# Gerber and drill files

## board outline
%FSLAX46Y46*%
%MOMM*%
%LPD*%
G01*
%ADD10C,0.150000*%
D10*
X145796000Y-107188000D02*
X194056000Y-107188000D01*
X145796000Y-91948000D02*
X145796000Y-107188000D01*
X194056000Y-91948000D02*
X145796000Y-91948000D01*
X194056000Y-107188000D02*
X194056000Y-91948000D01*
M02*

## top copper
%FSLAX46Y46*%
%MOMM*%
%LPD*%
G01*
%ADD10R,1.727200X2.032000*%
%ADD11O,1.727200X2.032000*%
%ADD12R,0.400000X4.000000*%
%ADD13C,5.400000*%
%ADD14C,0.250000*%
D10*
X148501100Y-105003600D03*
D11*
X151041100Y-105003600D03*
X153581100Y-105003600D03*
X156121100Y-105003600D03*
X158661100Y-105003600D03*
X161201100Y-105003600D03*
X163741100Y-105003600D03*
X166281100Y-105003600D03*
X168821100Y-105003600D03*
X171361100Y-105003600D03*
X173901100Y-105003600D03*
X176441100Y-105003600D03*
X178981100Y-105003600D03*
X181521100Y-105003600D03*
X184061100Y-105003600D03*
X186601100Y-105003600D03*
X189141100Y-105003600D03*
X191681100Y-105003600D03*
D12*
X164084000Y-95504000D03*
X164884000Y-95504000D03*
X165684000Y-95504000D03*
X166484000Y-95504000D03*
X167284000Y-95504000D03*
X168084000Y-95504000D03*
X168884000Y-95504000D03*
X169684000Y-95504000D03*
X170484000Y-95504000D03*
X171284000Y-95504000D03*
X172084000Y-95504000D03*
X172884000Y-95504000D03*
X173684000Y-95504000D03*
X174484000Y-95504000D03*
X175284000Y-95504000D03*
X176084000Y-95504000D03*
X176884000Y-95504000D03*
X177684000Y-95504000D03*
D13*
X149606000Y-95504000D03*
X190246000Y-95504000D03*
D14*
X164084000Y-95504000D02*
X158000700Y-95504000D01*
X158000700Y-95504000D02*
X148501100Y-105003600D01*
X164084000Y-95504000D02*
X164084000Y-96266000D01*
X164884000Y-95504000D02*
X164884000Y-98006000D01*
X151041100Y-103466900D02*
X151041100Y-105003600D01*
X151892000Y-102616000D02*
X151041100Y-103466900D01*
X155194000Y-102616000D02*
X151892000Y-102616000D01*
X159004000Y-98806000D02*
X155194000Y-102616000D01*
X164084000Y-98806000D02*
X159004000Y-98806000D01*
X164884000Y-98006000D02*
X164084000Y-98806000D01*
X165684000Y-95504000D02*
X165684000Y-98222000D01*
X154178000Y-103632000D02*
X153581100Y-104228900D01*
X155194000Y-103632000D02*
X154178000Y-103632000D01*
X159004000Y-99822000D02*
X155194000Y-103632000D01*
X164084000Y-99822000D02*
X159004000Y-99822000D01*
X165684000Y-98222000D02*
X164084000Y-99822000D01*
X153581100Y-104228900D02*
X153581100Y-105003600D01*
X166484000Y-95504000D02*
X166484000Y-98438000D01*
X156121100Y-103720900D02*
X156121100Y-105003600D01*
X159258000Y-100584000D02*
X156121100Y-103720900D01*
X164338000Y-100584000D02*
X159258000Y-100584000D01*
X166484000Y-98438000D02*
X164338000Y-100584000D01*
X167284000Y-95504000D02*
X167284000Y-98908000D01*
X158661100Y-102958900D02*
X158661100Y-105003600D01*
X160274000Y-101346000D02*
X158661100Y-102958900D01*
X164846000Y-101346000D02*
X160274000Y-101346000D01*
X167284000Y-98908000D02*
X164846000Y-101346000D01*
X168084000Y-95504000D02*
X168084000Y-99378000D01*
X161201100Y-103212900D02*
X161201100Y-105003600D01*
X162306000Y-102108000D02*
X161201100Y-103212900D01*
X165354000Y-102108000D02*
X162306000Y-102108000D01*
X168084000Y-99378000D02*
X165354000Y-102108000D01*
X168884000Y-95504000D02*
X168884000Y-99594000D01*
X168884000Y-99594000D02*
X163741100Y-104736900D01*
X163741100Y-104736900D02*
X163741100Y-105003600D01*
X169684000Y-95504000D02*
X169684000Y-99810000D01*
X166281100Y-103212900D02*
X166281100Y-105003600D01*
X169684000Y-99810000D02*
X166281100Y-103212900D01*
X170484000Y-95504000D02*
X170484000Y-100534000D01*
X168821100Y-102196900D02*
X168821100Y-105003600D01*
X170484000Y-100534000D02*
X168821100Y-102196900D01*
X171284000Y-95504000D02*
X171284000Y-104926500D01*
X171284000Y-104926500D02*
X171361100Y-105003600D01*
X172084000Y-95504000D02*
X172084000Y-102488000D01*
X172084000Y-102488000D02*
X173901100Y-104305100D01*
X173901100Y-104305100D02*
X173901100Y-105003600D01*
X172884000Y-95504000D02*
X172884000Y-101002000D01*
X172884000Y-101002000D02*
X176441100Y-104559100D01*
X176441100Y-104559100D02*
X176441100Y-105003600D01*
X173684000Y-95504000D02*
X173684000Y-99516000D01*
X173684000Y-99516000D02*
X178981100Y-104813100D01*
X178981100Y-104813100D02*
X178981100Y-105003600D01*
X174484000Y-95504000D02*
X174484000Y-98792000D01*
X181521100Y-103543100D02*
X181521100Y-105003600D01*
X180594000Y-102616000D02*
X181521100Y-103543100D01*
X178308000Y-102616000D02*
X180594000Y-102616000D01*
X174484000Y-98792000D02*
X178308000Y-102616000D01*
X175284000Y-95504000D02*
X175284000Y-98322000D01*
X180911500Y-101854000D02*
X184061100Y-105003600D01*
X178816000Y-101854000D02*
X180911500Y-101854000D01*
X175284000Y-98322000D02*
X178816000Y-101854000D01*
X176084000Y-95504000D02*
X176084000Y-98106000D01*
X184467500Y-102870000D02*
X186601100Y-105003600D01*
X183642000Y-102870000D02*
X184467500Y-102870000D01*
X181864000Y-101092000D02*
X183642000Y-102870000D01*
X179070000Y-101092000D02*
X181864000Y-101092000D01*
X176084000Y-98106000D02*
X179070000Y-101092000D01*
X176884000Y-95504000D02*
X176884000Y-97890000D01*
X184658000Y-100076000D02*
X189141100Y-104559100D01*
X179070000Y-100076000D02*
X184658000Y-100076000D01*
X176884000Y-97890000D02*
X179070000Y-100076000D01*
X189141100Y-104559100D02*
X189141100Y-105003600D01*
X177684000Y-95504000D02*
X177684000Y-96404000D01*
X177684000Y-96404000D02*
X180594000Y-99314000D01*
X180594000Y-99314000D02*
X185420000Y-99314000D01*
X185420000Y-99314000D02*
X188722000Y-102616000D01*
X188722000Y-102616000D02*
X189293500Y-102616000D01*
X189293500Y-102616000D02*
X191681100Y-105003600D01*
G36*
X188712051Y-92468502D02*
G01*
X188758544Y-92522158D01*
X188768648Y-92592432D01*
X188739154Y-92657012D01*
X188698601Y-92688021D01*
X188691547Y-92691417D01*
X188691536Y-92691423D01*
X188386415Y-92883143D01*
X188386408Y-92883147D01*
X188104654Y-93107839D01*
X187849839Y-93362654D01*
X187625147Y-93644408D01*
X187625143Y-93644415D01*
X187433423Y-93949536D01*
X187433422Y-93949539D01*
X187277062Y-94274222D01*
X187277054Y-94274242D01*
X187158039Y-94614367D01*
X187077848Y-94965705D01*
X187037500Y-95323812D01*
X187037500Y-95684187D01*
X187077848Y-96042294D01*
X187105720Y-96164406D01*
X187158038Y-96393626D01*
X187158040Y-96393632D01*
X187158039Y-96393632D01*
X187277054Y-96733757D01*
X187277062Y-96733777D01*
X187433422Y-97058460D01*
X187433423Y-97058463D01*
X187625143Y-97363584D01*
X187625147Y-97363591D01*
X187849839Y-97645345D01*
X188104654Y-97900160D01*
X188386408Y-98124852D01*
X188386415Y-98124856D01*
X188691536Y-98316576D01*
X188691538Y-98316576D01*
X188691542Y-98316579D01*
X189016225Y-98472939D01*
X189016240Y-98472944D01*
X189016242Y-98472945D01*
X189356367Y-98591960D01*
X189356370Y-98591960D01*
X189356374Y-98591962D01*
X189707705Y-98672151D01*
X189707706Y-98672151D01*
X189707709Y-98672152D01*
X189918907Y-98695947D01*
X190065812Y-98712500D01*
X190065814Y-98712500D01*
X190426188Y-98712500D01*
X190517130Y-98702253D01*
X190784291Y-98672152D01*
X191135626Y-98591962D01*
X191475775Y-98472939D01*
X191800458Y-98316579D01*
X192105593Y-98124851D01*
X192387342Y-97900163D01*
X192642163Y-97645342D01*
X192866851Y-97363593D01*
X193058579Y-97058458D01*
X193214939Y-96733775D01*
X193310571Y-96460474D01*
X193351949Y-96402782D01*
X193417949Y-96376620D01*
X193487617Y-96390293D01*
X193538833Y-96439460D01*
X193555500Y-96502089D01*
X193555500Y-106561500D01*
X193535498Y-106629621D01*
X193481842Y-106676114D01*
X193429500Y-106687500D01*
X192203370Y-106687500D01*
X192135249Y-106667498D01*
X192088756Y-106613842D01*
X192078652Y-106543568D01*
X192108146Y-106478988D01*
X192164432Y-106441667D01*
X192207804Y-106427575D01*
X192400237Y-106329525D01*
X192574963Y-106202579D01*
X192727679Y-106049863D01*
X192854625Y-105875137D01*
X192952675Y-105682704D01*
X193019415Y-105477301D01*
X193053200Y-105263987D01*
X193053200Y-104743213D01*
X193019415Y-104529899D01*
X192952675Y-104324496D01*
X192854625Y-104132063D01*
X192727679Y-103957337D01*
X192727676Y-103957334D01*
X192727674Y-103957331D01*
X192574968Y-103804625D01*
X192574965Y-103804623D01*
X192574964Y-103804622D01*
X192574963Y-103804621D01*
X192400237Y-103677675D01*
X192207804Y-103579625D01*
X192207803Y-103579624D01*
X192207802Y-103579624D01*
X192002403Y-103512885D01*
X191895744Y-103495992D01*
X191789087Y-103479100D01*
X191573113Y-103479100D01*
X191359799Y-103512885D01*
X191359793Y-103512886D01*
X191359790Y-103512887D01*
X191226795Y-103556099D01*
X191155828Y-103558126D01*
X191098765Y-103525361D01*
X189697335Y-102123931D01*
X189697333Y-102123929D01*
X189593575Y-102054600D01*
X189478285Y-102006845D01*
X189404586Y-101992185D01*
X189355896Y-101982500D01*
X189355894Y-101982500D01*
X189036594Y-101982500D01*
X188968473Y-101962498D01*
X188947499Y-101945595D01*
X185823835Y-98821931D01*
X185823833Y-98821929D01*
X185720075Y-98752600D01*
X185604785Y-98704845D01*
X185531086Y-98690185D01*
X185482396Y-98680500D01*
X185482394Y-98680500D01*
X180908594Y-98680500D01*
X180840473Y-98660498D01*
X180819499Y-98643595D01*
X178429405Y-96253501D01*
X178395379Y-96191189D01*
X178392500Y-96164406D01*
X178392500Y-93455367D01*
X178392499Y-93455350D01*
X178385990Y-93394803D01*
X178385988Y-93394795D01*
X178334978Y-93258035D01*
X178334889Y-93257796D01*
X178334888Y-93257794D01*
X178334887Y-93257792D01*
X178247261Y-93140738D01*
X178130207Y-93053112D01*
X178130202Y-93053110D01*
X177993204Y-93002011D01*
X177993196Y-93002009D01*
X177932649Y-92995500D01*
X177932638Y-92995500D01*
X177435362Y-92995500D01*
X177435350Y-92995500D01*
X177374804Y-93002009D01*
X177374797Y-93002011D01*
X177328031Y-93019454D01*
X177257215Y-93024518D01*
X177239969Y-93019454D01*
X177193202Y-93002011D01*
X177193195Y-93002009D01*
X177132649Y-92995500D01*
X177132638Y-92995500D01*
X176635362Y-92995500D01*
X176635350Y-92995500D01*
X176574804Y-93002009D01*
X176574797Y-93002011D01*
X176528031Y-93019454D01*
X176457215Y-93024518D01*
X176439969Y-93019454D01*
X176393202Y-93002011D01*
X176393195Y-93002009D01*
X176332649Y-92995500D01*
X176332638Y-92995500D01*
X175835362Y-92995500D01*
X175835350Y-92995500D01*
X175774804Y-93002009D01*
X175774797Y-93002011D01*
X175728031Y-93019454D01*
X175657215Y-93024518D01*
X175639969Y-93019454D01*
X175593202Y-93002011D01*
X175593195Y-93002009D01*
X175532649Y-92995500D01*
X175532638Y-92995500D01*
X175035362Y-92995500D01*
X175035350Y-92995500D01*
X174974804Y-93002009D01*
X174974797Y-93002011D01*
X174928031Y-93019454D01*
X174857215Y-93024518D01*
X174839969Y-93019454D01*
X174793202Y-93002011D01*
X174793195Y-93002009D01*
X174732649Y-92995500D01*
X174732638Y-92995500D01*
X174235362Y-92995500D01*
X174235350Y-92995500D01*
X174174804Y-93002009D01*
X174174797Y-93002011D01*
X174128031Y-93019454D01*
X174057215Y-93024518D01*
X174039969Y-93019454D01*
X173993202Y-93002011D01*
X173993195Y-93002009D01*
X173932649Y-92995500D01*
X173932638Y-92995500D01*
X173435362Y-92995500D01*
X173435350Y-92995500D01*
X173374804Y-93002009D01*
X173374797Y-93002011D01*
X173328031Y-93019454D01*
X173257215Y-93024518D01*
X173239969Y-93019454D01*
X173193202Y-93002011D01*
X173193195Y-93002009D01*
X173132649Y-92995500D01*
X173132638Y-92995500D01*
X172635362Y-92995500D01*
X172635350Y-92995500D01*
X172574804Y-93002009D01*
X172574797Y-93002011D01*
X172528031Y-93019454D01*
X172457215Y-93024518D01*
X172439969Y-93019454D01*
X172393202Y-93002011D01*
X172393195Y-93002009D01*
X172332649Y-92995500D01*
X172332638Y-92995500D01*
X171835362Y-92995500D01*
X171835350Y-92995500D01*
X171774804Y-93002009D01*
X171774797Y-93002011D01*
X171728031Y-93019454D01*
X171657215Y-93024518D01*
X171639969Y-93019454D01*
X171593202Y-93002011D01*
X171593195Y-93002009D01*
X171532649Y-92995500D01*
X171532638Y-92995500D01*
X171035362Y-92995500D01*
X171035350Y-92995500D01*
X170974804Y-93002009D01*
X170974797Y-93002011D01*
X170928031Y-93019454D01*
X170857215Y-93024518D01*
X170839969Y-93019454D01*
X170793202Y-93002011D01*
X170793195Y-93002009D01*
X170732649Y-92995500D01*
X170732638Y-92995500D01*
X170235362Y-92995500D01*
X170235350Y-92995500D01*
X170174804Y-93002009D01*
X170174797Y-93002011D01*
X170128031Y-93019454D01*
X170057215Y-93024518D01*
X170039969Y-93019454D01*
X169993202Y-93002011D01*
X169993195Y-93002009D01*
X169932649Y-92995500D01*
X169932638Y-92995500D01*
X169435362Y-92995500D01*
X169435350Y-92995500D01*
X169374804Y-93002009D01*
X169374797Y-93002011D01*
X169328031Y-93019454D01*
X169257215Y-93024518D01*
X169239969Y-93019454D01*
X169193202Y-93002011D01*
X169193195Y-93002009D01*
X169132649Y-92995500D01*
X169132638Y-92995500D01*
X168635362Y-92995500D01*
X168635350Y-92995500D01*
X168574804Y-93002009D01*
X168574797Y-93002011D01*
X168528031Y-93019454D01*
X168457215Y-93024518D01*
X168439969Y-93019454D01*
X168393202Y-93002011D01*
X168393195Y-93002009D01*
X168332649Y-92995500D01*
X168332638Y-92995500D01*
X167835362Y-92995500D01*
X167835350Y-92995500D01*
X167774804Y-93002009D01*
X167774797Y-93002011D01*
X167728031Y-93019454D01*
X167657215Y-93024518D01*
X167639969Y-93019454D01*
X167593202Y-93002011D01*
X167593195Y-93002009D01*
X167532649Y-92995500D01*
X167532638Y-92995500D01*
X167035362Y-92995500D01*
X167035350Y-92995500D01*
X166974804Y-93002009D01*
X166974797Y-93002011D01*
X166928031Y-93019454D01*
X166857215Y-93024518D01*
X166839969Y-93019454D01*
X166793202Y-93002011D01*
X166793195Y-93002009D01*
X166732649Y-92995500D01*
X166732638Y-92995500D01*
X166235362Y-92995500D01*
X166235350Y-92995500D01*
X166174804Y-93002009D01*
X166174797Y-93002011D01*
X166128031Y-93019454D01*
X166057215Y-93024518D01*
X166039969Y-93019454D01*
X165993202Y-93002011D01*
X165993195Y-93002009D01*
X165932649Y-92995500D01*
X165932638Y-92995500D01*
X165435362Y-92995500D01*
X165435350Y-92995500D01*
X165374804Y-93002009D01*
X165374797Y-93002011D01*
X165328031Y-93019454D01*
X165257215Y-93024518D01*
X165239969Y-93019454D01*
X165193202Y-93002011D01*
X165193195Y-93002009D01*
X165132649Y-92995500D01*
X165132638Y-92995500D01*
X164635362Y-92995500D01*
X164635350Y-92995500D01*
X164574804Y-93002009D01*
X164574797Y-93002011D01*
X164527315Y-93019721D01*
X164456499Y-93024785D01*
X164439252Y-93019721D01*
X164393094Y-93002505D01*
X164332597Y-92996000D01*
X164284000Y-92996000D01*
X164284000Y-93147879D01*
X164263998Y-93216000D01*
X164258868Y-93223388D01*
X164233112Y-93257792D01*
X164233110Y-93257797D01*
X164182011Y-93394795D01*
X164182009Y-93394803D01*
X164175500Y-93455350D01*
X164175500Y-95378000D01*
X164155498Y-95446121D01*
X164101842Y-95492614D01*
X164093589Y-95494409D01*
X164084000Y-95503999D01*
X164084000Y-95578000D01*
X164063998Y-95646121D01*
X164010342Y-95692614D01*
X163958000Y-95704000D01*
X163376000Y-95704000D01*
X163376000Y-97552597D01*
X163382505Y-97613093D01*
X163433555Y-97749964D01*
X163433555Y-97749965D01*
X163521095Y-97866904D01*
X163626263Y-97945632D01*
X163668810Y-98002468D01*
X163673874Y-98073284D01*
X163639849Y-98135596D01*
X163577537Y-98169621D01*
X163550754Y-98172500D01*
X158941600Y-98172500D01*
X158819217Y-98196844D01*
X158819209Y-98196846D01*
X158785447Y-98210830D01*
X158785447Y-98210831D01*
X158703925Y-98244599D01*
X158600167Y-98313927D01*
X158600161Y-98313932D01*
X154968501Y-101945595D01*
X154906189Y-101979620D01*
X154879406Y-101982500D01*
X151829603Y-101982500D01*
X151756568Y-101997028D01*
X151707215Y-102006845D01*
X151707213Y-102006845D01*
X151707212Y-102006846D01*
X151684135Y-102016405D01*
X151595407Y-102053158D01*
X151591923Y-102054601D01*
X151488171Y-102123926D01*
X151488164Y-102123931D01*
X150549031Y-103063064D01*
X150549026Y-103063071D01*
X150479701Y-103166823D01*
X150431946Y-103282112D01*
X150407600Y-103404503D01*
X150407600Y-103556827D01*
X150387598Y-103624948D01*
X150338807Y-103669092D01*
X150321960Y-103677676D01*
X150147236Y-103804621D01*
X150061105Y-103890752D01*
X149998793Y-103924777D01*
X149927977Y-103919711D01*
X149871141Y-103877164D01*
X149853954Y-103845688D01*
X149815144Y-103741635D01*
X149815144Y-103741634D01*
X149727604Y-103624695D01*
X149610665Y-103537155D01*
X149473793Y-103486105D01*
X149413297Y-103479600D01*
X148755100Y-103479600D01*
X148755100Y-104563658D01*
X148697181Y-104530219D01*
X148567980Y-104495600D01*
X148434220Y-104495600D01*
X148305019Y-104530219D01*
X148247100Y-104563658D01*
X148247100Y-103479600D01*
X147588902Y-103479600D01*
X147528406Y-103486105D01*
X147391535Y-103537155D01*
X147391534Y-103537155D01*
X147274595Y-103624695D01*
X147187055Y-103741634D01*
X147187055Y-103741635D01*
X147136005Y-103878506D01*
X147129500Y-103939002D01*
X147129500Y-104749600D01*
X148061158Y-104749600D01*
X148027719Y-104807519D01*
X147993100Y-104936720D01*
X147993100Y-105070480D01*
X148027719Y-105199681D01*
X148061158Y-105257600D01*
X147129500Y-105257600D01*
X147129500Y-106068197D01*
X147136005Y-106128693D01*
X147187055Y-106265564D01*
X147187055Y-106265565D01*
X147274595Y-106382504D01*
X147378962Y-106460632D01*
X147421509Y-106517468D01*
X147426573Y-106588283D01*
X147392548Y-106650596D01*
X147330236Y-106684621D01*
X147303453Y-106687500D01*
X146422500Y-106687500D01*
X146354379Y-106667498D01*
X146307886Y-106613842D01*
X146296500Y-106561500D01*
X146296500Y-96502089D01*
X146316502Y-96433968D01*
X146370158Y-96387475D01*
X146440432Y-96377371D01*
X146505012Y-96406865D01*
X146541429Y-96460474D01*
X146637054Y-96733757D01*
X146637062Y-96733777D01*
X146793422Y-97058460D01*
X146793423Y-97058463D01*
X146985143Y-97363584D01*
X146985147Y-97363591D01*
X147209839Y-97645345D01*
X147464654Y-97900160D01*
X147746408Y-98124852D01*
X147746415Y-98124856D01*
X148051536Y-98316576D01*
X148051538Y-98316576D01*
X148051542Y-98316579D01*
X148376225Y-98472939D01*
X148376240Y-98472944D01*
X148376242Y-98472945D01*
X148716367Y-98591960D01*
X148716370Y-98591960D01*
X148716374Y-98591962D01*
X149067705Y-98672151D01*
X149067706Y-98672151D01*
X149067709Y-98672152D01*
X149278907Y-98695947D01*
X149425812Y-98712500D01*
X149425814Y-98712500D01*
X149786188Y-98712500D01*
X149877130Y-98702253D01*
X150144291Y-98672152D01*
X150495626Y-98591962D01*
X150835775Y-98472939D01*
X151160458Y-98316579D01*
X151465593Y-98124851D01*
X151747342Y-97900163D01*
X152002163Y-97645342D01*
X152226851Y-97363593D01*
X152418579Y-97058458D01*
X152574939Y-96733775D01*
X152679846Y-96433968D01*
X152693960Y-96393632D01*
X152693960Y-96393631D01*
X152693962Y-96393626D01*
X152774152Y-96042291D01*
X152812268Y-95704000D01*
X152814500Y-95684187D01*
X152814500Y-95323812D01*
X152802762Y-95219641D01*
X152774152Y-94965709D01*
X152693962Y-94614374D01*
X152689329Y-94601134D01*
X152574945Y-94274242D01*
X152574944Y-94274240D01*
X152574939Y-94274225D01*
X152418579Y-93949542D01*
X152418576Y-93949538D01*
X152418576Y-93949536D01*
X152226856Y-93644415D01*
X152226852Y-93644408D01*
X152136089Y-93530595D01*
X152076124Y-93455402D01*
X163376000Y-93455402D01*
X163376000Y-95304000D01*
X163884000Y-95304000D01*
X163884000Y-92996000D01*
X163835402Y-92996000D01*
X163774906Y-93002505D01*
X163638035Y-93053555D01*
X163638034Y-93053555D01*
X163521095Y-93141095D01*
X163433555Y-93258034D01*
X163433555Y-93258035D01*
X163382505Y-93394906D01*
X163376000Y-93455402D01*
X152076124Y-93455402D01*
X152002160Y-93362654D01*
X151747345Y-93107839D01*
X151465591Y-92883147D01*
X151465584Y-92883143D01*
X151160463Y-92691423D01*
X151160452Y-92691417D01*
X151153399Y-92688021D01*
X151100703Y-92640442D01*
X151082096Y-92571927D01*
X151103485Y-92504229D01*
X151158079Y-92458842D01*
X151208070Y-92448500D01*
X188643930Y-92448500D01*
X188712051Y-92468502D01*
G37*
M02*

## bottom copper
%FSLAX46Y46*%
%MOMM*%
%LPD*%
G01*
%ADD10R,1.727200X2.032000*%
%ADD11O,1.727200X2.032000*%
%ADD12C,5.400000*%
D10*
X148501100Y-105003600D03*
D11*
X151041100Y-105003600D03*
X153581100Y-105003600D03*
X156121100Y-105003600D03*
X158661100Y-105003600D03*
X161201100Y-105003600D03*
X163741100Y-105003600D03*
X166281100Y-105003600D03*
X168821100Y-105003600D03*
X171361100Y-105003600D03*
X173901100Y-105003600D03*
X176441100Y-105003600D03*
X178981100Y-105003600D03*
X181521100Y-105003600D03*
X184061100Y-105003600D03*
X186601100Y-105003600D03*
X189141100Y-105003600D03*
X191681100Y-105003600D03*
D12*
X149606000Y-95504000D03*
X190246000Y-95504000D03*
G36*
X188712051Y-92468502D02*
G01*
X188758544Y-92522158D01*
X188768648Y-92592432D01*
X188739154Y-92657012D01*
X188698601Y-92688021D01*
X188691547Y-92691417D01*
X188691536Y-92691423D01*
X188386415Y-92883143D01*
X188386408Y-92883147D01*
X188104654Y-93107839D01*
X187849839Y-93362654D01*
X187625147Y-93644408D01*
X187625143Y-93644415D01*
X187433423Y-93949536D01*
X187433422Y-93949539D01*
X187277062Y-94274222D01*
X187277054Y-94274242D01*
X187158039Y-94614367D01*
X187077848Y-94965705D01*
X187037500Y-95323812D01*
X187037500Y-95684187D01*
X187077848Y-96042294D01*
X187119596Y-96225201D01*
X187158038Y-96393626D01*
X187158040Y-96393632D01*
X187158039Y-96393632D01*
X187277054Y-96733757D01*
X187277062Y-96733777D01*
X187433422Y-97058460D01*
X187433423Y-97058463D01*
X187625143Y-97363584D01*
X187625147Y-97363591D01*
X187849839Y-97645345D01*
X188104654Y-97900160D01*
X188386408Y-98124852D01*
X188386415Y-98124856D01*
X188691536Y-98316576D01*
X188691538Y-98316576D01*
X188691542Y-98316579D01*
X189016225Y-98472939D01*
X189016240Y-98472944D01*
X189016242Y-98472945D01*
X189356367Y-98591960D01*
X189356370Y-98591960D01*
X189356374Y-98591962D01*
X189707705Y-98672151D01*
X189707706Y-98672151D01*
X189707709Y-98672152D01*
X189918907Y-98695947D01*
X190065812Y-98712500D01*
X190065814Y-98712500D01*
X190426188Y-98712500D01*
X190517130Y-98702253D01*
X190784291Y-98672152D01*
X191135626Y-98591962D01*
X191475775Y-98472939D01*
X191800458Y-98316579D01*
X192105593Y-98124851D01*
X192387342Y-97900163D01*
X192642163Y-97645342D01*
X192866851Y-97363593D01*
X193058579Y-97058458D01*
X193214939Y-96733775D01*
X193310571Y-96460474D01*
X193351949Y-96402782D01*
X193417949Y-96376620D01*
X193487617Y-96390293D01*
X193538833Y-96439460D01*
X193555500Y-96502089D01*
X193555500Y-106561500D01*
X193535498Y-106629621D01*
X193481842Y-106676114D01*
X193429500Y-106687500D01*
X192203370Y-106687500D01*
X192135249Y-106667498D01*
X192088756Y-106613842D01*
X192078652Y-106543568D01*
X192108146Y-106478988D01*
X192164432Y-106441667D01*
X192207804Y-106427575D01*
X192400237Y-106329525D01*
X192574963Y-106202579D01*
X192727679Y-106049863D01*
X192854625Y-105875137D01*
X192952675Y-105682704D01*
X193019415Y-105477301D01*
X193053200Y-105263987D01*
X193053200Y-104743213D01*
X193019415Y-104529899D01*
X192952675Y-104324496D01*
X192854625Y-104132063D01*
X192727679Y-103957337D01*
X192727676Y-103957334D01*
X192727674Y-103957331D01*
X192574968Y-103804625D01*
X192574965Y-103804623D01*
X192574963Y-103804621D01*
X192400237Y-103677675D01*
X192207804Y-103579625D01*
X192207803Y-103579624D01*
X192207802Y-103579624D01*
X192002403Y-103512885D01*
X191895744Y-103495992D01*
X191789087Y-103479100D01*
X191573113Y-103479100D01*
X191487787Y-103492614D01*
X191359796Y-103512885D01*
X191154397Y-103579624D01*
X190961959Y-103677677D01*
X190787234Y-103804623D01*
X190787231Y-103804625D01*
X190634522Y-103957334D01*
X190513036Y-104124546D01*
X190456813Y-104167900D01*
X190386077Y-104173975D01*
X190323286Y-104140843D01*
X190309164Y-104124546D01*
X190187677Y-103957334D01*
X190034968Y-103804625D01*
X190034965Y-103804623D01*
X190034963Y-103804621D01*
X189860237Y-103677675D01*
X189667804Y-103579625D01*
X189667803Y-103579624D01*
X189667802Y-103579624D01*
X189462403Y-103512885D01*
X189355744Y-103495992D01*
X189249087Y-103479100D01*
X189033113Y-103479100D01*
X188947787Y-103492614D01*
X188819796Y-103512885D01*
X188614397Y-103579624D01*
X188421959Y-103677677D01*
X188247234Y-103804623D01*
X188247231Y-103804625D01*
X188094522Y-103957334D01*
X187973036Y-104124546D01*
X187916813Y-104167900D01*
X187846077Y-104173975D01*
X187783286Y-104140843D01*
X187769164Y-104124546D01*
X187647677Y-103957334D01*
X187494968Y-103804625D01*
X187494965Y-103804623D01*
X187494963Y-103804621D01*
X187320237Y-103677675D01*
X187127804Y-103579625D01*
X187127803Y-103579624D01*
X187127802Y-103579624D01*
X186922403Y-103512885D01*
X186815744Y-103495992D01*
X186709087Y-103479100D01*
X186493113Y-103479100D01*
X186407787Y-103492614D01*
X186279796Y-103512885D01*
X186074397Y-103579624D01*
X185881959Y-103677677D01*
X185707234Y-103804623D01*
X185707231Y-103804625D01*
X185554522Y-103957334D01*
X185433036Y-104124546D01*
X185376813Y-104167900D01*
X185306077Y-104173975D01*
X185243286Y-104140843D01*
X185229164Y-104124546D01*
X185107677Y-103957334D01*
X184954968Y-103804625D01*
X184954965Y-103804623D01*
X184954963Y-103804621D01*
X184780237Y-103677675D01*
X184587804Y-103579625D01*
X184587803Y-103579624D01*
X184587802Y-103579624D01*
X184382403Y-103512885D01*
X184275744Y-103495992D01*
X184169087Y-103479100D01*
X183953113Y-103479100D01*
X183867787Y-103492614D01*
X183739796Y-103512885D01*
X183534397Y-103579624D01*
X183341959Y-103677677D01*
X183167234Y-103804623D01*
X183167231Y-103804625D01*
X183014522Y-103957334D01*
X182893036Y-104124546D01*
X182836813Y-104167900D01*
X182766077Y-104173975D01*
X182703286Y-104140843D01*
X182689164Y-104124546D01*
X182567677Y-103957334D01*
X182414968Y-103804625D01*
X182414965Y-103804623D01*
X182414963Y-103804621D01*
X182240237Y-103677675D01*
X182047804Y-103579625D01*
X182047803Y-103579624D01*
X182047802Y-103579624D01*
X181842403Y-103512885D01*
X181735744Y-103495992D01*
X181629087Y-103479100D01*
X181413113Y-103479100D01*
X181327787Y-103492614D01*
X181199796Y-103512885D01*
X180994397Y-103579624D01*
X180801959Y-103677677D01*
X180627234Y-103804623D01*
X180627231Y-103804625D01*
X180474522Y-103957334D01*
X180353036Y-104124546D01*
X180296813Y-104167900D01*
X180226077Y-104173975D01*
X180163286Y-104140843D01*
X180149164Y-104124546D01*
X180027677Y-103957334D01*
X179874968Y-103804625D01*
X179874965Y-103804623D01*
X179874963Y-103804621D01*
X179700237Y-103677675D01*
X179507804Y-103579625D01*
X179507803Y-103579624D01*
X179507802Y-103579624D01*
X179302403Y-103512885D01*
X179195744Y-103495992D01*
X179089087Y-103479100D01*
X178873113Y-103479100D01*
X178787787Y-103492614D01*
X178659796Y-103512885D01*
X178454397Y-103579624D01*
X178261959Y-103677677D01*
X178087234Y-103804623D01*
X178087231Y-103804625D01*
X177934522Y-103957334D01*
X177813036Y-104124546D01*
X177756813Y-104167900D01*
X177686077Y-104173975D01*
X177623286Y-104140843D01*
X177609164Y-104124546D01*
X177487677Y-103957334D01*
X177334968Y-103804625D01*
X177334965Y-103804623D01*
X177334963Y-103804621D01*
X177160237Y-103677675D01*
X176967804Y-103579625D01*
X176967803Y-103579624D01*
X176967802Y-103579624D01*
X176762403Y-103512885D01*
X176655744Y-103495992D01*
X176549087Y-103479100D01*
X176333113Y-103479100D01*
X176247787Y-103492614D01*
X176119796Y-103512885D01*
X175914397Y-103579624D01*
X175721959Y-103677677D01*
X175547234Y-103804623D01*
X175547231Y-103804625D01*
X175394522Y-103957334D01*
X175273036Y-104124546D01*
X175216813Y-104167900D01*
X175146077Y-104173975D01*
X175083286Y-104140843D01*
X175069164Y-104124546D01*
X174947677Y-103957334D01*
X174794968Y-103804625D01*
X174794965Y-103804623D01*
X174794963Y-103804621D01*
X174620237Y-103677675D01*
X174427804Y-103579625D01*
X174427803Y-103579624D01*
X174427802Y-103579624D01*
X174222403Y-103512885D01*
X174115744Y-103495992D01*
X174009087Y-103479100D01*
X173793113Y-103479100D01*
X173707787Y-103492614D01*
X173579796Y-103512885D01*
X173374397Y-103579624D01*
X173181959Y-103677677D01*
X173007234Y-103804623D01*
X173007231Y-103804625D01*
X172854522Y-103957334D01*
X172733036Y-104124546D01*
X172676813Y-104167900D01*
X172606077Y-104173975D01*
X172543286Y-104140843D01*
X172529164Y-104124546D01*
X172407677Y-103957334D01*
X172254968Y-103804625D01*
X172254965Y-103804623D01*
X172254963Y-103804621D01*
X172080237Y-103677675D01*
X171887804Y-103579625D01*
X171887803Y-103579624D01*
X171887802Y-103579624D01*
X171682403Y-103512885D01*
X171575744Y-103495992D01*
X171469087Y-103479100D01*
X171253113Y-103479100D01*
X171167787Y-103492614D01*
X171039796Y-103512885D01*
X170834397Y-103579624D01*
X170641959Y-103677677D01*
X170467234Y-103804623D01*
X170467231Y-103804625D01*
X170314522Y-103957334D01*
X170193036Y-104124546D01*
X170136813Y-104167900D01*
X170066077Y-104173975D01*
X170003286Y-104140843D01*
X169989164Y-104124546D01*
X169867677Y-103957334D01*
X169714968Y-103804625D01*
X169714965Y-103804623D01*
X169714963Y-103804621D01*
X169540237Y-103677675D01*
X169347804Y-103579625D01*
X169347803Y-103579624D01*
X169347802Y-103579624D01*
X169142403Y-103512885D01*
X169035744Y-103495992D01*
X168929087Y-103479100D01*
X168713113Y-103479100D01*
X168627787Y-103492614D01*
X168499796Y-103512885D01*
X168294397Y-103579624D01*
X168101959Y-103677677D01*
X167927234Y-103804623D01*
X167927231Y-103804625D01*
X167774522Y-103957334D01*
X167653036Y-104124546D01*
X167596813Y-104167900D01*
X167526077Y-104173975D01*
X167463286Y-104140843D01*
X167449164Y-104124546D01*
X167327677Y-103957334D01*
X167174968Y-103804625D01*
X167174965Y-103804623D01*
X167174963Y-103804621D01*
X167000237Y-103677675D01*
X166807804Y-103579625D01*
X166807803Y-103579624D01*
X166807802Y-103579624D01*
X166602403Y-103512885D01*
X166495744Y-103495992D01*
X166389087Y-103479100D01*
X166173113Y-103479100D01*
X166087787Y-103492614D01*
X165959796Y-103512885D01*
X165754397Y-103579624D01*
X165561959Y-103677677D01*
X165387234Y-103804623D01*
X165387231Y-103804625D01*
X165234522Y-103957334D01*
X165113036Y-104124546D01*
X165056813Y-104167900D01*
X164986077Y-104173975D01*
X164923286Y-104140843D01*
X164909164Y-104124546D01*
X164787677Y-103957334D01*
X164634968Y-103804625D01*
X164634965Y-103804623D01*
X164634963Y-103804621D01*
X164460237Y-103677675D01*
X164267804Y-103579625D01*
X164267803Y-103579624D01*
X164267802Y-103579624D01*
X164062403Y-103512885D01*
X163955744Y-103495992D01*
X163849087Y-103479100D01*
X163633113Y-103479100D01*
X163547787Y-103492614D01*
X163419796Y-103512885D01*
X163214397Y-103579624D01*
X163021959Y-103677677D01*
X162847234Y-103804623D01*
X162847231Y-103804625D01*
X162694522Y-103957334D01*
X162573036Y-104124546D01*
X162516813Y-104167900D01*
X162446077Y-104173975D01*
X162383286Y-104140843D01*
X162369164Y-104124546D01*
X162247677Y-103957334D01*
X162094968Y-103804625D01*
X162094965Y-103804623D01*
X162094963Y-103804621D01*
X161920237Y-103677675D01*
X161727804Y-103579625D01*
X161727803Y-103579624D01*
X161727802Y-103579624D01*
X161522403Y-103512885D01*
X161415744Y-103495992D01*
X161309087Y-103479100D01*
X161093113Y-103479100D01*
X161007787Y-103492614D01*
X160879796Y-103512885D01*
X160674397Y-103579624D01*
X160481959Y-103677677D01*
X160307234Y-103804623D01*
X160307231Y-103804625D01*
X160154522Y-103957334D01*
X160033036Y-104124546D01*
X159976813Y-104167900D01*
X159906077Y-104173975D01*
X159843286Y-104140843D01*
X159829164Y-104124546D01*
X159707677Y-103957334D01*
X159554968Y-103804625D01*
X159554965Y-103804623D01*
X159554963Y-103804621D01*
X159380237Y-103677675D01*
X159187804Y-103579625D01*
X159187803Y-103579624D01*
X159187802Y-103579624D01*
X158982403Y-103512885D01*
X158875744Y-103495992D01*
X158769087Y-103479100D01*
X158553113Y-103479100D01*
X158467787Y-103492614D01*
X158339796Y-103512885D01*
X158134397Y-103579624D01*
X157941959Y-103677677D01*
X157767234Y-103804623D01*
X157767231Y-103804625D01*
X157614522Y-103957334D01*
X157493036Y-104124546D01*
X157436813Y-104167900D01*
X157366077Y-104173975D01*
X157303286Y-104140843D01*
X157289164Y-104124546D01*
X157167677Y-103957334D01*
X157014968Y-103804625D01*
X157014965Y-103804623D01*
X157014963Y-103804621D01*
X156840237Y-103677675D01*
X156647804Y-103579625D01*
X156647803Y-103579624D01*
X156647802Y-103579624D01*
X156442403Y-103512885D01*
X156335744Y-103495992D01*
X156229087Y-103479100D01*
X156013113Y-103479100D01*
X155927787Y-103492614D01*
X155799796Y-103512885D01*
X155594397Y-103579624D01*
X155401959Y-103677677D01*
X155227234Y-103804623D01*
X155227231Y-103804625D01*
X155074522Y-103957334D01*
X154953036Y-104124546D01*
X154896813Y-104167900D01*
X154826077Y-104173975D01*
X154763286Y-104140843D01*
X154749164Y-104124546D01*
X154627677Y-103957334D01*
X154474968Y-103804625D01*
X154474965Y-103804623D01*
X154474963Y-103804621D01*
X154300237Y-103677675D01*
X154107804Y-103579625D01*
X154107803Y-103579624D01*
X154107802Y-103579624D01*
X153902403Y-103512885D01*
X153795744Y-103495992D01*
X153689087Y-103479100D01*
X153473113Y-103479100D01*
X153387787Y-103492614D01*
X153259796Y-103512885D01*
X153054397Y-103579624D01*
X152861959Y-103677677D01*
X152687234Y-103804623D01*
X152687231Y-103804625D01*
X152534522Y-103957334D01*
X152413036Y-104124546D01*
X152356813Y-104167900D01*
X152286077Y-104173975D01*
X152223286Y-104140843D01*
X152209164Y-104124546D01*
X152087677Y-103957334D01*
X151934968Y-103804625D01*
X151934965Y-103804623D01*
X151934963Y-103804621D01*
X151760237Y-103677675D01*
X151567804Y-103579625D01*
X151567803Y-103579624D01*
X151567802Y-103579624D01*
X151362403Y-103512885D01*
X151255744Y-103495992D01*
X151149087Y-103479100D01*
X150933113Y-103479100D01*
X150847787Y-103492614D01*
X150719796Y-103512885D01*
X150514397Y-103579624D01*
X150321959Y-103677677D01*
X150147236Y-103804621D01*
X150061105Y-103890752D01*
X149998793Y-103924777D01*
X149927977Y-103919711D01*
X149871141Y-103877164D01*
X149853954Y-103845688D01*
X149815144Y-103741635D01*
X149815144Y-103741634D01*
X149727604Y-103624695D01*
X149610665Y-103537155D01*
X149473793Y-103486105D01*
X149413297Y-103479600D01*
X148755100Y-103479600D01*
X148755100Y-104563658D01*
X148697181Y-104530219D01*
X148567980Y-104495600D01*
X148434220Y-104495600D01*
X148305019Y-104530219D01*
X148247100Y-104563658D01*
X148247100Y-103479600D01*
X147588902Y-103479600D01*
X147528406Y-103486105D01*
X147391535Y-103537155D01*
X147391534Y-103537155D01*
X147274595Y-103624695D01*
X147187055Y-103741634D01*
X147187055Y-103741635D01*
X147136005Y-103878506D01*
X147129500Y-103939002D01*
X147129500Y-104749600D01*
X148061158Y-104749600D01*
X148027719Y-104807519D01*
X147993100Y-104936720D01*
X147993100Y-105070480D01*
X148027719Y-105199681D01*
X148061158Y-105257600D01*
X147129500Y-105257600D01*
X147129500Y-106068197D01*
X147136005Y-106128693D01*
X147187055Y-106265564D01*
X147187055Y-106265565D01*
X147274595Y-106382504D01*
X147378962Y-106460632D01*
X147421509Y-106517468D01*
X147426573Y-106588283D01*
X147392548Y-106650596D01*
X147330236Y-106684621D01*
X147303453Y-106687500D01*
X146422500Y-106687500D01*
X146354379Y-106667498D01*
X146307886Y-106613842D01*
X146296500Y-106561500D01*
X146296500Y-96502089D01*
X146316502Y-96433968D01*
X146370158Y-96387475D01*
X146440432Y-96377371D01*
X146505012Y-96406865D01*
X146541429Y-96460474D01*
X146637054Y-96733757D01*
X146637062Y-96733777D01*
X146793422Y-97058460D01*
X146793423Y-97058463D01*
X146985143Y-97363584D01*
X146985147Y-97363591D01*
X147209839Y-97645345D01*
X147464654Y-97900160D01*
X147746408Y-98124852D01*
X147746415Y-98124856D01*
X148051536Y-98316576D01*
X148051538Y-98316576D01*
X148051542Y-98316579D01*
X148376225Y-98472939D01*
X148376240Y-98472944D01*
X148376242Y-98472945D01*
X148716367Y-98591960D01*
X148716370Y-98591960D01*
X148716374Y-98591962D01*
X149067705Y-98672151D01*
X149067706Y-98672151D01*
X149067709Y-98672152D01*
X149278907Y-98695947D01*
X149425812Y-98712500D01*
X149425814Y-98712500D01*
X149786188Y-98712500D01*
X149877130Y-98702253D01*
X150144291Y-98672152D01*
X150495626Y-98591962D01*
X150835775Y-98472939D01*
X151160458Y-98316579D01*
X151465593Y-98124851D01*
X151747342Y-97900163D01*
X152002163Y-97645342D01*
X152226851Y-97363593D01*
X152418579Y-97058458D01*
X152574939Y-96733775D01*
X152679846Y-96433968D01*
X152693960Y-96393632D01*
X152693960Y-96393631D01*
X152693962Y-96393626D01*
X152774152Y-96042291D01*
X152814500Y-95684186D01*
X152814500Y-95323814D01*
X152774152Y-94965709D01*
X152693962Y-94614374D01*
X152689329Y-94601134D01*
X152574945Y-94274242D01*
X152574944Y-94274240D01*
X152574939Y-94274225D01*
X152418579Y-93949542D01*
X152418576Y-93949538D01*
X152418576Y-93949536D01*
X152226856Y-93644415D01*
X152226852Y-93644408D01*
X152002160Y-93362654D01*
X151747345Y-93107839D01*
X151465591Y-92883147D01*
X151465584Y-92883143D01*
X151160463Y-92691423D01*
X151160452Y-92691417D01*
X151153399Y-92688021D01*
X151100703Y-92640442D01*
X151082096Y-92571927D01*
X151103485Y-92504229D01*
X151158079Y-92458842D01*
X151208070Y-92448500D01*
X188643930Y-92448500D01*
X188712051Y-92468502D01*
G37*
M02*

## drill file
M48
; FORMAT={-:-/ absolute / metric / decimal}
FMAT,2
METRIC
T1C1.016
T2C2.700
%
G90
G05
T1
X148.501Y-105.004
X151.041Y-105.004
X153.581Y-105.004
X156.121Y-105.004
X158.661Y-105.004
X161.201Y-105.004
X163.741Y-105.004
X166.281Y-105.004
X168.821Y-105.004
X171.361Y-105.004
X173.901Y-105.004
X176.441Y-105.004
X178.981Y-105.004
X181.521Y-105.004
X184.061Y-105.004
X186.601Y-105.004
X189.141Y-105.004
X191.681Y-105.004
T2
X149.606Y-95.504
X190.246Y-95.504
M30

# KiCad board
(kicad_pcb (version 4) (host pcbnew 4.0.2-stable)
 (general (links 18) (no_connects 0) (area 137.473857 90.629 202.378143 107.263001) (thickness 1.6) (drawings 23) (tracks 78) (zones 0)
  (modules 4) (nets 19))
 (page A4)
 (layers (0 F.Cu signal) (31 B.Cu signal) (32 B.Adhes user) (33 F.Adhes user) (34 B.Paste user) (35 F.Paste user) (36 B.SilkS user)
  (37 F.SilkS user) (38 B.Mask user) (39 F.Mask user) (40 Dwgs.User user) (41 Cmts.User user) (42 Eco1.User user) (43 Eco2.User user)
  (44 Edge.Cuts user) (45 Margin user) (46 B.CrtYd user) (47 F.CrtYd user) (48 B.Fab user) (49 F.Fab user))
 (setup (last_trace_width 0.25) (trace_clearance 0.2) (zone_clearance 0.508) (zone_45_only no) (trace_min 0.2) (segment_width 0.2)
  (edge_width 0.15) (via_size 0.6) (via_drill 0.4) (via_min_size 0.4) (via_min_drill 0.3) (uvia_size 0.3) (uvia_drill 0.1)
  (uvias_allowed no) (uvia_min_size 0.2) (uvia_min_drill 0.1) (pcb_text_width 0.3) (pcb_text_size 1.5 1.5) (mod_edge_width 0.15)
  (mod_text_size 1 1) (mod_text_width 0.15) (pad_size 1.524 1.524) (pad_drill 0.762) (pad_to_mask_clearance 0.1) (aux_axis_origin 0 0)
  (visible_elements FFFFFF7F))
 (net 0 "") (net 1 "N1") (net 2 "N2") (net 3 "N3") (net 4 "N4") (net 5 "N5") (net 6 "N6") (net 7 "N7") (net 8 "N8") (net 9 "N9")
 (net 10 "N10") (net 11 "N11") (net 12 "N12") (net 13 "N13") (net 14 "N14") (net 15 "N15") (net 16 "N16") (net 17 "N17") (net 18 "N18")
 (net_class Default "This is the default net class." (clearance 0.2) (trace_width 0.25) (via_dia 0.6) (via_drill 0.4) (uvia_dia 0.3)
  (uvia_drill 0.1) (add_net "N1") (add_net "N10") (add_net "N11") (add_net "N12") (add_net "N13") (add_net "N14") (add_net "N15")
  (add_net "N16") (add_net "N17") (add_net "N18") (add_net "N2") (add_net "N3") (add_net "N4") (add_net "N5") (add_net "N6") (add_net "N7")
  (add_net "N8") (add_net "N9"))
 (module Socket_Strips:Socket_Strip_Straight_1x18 (layer F.Cu) (at 148.5011 105.0036)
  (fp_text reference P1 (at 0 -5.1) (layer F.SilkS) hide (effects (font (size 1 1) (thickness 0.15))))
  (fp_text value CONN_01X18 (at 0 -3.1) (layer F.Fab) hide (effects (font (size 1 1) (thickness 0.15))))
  (pad 1 thru_hole rect (at 0 0) (size 1.7272 2.032) (drill 1.016) (layers *.Cu *.Mask) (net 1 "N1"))
  (pad 2 thru_hole oval (at 2.54 0) (size 1.7272 2.032) (drill 1.016) (layers *.Cu *.Mask) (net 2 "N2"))
  (pad 3 thru_hole oval (at 5.08 0) (size 1.7272 2.032) (drill 1.016) (layers *.Cu *.Mask) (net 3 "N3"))
  (pad 4 thru_hole oval (at 7.62 0) (size 1.7272 2.032) (drill 1.016) (layers *.Cu *.Mask) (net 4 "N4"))
  (pad 5 thru_hole oval (at 10.16 0) (size 1.7272 2.032) (drill 1.016) (layers *.Cu *.Mask) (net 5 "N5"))
  (pad 6 thru_hole oval (at 12.7 0) (size 1.7272 2.032) (drill 1.016) (layers *.Cu *.Mask) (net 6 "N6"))
  (pad 7 thru_hole oval (at 15.24 0) (size 1.7272 2.032) (drill 1.016) (layers *.Cu *.Mask) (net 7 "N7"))
  (pad 8 thru_hole oval (at 17.78 0) (size 1.7272 2.032) (drill 1.016) (layers *.Cu *.Mask) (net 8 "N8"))
  (pad 9 thru_hole oval (at 20.32 0) (size 1.7272 2.032) (drill 1.016) (layers *.Cu *.Mask) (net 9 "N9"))
  (pad 10 thru_hole oval (at 22.86 0) (size 1.7272 2.032) (drill 1.016) (layers *.Cu *.Mask) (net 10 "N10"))
  (pad 11 thru_hole oval (at 25.4 0) (size 1.7272 2.032) (drill 1.016) (layers *.Cu *.Mask) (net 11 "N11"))
  (pad 12 thru_hole oval (at 27.94 0) (size 1.7272 2.032) (drill 1.016) (layers *.Cu *.Mask) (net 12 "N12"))
  (pad 13 thru_hole oval (at 30.48 0) (size 1.7272 2.032) (drill 1.016) (layers *.Cu *.Mask) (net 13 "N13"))
  (pad 14 thru_hole oval (at 33.02 0) (size 1.7272 2.032) (drill 1.016) (layers *.Cu *.Mask) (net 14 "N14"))
  (pad 15 thru_hole oval (at 35.56 0) (size 1.7272 2.032) (drill 1.016) (layers *.Cu *.Mask) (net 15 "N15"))
  (pad 16 thru_hole oval (at 38.1 0) (size 1.7272 2.032) (drill 1.016) (layers *.Cu *.Mask) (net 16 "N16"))
  (pad 17 thru_hole oval (at 40.64 0) (size 1.7272 2.032) (drill 1.016) (layers *.Cu *.Mask) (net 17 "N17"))
  (pad 18 thru_hole oval (at 43.18 0) (size 1.7272 2.032) (drill 1.016) (layers *.Cu *.Mask) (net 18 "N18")))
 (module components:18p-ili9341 (layer F.Cu) (at 164.084 95.504)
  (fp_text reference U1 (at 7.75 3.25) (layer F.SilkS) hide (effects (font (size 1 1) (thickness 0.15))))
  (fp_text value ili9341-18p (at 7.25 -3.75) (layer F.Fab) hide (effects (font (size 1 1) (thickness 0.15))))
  (pad 1 smd rect (at 0 0) (size 0.4 4) (layers F.Cu F.Paste F.Mask) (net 1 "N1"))
  (pad 2 smd rect (at 0.8 0) (size 0.4 4) (layers F.Cu F.Paste F.Mask) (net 2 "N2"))
  (pad 3 smd rect (at 1.6 0) (size 0.4 4) (layers F.Cu F.Paste F.Mask) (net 3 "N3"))
  (pad 4 smd rect (at 2.4 0) (size 0.4 4) (layers F.Cu F.Paste F.Mask) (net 4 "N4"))
  (pad 5 smd rect (at 3.2 0) (size 0.4 4) (layers F.Cu F.Paste F.Mask) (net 5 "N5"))
  (pad 6 smd rect (at 4 0) (size 0.4 4) (layers F.Cu F.Paste F.Mask) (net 6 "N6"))
  (pad 7 smd rect (at 4.8 0) (size 0.4 4) (layers F.Cu F.Paste F.Mask) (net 7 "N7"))
  (pad 8 smd rect (at 5.6 0) (size 0.4 4) (layers F.Cu F.Paste F.Mask) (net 8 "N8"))
  (pad 9 smd rect (at 6.4 0) (size 0.4 4) (layers F.Cu F.Paste F.Mask) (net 9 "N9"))
  (pad 10 smd rect (at 7.2 0) (size 0.4 4) (layers F.Cu F.Paste F.Mask) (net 10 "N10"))
  (pad 11 smd rect (at 8 0) (size 0.4 4) (layers F.Cu F.Paste F.Mask) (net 11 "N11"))
  (pad 12 smd rect (at 8.8 0) (size 0.4 4) (layers F.Cu F.Paste F.Mask) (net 12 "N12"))
  (pad 13 smd rect (at 9.6 0) (size 0.4 4) (layers F.Cu F.Paste F.Mask) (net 13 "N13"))
  (pad 14 smd rect (at 10.4 0) (size 0.4 4) (layers F.Cu F.Paste F.Mask) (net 14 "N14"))
  (pad 15 smd rect (at 11.2 0) (size 0.4 4) (layers F.Cu F.Paste F.Mask) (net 15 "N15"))
  (pad 16 smd rect (at 12 0) (size 0.4 4) (layers F.Cu F.Paste F.Mask) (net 16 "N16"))
  (pad 17 smd rect (at 12.8 0) (size 0.4 4) (layers F.Cu F.Paste F.Mask) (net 17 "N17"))
  (pad 18 smd rect (at 13.6 0) (size 0.4 4) (layers F.Cu F.Paste F.Mask) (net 18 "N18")))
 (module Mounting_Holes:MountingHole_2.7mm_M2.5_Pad (layer F.Cu) (at 149.606 95.504)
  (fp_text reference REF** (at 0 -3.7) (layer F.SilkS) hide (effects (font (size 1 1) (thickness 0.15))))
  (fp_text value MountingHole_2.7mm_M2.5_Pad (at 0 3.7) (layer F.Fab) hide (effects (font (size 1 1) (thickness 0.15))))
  (pad 1 thru_hole circle (at 0 0) (size 5.4 5.4) (drill 2.7) (layers *.Cu *.Mask)))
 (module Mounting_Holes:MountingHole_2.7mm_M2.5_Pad (layer F.Cu) (at 190.246 95.504)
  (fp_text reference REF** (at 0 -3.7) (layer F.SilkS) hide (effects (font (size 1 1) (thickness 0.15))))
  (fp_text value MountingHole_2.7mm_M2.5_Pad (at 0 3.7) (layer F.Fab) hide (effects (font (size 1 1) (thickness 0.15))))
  (pad 1 thru_hole circle (at 0 0) (size 5.4 5.4) (drill 2.7) (layers *.Cu *.Mask)))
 (gr_line (start 145.796 107.188) (end 194.056 107.188) (angle 90) (layer Edge.Cuts) (width 0.15))
 (gr_line (start 145.796 91.948) (end 145.796 107.188) (angle 90) (layer Edge.Cuts) (width 0.15))
 (gr_line (start 194.056 91.948) (end 145.796 91.948) (angle 90) (layer Edge.Cuts) (width 0.15))
 (gr_line (start 194.056 107.188) (end 194.056 91.948) (angle 90) (layer Edge.Cuts) (width 0.15))
 (segment (start 164.084 95.504) (end 158.0007 95.504) (width 0.25) (layer F.Cu) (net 1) (status 400000))
 (segment (start 158.0007 95.504) (end 148.5011 105.0036) (width 0.25) (layer F.Cu) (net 1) (status 800000))
 (segment (start 164.084 95.504) (end 164.084 96.266) (width 0.25) (layer F.Cu) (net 1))
 (segment (start 164.884 95.504) (end 164.884 98.006) (width 0.25) (layer F.Cu) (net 2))
 (segment (start 151.0411 103.4669) (end 151.0411 105.0036) (width 0.25) (layer F.Cu) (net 2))
 (segment (start 151.892 102.616) (end 151.0411 103.4669) (width 0.25) (layer F.Cu) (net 2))
 (segment (start 155.194 102.616) (end 151.892 102.616) (width 0.25) (layer F.Cu) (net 2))
 (segment (start 159.004 98.806) (end 155.194 102.616) (width 0.25) (layer F.Cu) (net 2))
 (segment (start 164.084 98.806) (end 159.004 98.806) (width 0.25) (layer F.Cu) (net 2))
 (segment (start 164.884 98.006) (end 164.084 98.806) (width 0.25) (layer F.Cu) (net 2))
 (segment (start 165.684 95.504) (end 165.684 98.222) (width 0.25) (layer F.Cu) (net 3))
 (segment (start 154.178 103.632) (end 153.5811 104.2289) (width 0.25) (layer F.Cu) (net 3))
 (segment (start 155.194 103.632) (end 154.178 103.632) (width 0.25) (layer F.Cu) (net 3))
 (segment (start 159.004 99.822) (end 155.194 103.632) (width 0.25) (layer F.Cu) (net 3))
 (segment (start 164.084 99.822) (end 159.004 99.822) (width 0.25) (layer F.Cu) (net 3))
 (segment (start 165.684 98.222) (end 164.084 99.822) (width 0.25) (layer F.Cu) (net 3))
 (segment (start 153.5811 104.2289) (end 153.5811 105.0036) (width 0.25) (layer F.Cu) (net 3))
 (segment (start 166.484 95.504) (end 166.484 98.438) (width 0.25) (layer F.Cu) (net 4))
 (segment (start 156.1211 103.7209) (end 156.1211 105.0036) (width 0.25) (layer F.Cu) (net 4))
 (segment (start 159.258 100.584) (end 156.1211 103.7209) (width 0.25) (layer F.Cu) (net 4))
 (segment (start 164.338 100.584) (end 159.258 100.584) (width 0.25) (layer F.Cu) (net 4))
 (segment (start 166.484 98.438) (end 164.338 100.584) (width 0.25) (layer F.Cu) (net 4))
 (segment (start 167.284 95.504) (end 167.284 98.908) (width 0.25) (layer F.Cu) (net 5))
 (segment (start 158.6611 102.9589) (end 158.6611 105.0036) (width 0.25) (layer F.Cu) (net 5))
 (segment (start 160.274 101.346) (end 158.6611 102.9589) (width 0.25) (layer F.Cu) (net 5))
 (segment (start 164.846 101.346) (end 160.274 101.346) (width 0.25) (layer F.Cu) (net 5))
 (segment (start 167.284 98.908) (end 164.846 101.346) (width 0.25) (layer F.Cu) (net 5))
 (segment (start 168.084 95.504) (end 168.084 99.378) (width 0.25) (layer F.Cu) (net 6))
 (segment (start 161.2011 103.2129) (end 161.2011 105.0036) (width 0.25) (layer F.Cu) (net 6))
 (segment (start 162.306 102.108) (end 161.2011 103.2129) (width 0.25) (layer F.Cu) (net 6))
 (segment (start 165.354 102.108) (end 162.306 102.108) (width 0.25) (layer F.Cu) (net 6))
 (segment (start 168.084 99.378) (end 165.354 102.108) (width 0.25) (layer F.Cu) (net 6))
 (segment (start 168.884 95.504) (end 168.884 99.594) (width 0.25) (layer F.Cu) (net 7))
 (segment (start 168.884 99.594) (end 163.7411 104.7369) (width 0.25) (layer F.Cu) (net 7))
 (segment (start 163.7411 104.7369) (end 163.7411 105.0036) (width 0.25) (layer F.Cu) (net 7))
 (segment (start 169.684 95.504) (end 169.684 99.81) (width 0.25) (layer F.Cu) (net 8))
 (segment (start 166.2811 103.2129) (end 166.2811 105.0036) (width 0.25) (layer F.Cu) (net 8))
 (segment (start 169.684 99.81) (end 166.2811 103.2129) (width 0.25) (layer F.Cu) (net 8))
 (segment (start 170.484 95.504) (end 170.484 100.534) (width 0.25) (layer F.Cu) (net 9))
 (segment (start 168.8211 102.1969) (end 168.8211 105.0036) (width 0.25) (layer F.Cu) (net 9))
 (segment (start 170.484 100.534) (end 168.8211 102.1969) (width 0.25) (layer F.Cu) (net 9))
 (segment (start 171.284 95.504) (end 171.284 104.9265) (width 0.25) (layer F.Cu) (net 10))
 (segment (start 171.284 104.9265) (end 171.3611 105.0036) (width 0.25) (layer F.Cu) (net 10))
 (segment (start 172.084 95.504) (end 172.084 102.488) (width 0.25) (layer F.Cu) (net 11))
 (segment (start 172.084 102.488) (end 173.9011 104.3051) (width 0.25) (layer F.Cu) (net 11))
 (segment (start 173.9011 104.3051) (end 173.9011 105.0036) (width 0.25) (layer F.Cu) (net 11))
 (segment (start 172.884 95.504) (end 172.884 101.002) (width 0.25) (layer F.Cu) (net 12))
 (segment (start 172.884 101.002) (end 176.4411 104.5591) (width 0.25) (layer F.Cu) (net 12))
 (segment (start 176.4411 104.5591) (end 176.4411 105.0036) (width 0.25) (layer F.Cu) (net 12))
 (segment (start 173.684 95.504) (end 173.684 99.516) (width 0.25) (layer F.Cu) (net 13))
 (segment (start 173.684 99.516) (end 178.9811 104.8131) (width 0.25) (layer F.Cu) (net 13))
 (segment (start 178.9811 104.8131) (end 178.9811 105.0036) (width 0.25) (layer F.Cu) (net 13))
 (segment (start 174.484 95.504) (end 174.484 98.792) (width 0.25) (layer F.Cu) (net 14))
 (segment (start 181.5211 103.5431) (end 181.5211 105.0036) (width 0.25) (layer F.Cu) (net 14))
 (segment (start 180.594 102.616) (end 181.5211 103.5431) (width 0.25) (layer F.Cu) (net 14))
 (segment (start 178.308 102.616) (end 180.594 102.616) (width 0.25) (layer F.Cu) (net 14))
 (segment (start 174.484 98.792) (end 178.308 102.616) (width 0.25) (layer F.Cu) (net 14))
 (segment (start 175.284 95.504) (end 175.284 98.322) (width 0.25) (layer F.Cu) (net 15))
 (segment (start 180.9115 101.854) (end 184.0611 105.0036) (width 0.25) (layer F.Cu) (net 15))
 (segment (start 178.816 101.854) (end 180.9115 101.854) (width 0.25) (layer F.Cu) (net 15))
 (segment (start 175.284 98.322) (end 178.816 101.854) (width 0.25) (layer F.Cu) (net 15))
 (segment (start 176.084 95.504) (end 176.084 98.106) (width 0.25) (layer F.Cu) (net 16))
 (segment (start 184.4675 102.87) (end 186.6011 105.0036) (width 0.25) (layer F.Cu) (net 16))
 (segment (start 183.642 102.87) (end 184.4675 102.87) (width 0.25) (layer F.Cu) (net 16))
 (segment (start 181.864 101.092) (end 183.642 102.87) (width 0.25) (layer F.Cu) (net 16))
 (segment (start 179.07 101.092) (end 181.864 101.092) (width 0.25) (layer F.Cu) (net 16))
 (segment (start 176.084 98.106) (end 179.07 101.092) (width 0.25) (layer F.Cu) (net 16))
 (segment (start 176.884 95.504) (end 176.884 97.89) (width 0.25) (layer F.Cu) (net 17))
 (segment (start 184.658 100.076) (end 189.1411 104.5591) (width 0.25) (layer F.Cu) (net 17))
 (segment (start 179.07 100.076) (end 184.658 100.076) (width 0.25) (layer F.Cu) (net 17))
 (segment (start 176.884 97.89) (end 179.07 100.076) (width 0.25) (layer F.Cu) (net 17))
 (segment (start 189.1411 104.5591) (end 189.1411 105.0036) (width 0.25) (layer F.Cu) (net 17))
 (segment (start 177.684 95.504) (end 177.684 96.404) (width 0.25) (layer F.Cu) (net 18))
 (segment (start 177.684 96.404) (end 180.594 99.314) (width 0.25) (layer F.Cu) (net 18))
 (segment (start 180.594 99.314) (end 185.42 99.314) (width 0.25) (layer F.Cu) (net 18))
 (segment (start 185.42 99.314) (end 188.722 102.616) (width 0.25) (layer F.Cu) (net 18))
 (segment (start 188.722 102.616) (end 189.2935 102.616) (width 0.25) (layer F.Cu) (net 18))
 (segment (start 189.2935 102.616) (end 191.6811 105.0036) (width 0.25) (layer F.Cu) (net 18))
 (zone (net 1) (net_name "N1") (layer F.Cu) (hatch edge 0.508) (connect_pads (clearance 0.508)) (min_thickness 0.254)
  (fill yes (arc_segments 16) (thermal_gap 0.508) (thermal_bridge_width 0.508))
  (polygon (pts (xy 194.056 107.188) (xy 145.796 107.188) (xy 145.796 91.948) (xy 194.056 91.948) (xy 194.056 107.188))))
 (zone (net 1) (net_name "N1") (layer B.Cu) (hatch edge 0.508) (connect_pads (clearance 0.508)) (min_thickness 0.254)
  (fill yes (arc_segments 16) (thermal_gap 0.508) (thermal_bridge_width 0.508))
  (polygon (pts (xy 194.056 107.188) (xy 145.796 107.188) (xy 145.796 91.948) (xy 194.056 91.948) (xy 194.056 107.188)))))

